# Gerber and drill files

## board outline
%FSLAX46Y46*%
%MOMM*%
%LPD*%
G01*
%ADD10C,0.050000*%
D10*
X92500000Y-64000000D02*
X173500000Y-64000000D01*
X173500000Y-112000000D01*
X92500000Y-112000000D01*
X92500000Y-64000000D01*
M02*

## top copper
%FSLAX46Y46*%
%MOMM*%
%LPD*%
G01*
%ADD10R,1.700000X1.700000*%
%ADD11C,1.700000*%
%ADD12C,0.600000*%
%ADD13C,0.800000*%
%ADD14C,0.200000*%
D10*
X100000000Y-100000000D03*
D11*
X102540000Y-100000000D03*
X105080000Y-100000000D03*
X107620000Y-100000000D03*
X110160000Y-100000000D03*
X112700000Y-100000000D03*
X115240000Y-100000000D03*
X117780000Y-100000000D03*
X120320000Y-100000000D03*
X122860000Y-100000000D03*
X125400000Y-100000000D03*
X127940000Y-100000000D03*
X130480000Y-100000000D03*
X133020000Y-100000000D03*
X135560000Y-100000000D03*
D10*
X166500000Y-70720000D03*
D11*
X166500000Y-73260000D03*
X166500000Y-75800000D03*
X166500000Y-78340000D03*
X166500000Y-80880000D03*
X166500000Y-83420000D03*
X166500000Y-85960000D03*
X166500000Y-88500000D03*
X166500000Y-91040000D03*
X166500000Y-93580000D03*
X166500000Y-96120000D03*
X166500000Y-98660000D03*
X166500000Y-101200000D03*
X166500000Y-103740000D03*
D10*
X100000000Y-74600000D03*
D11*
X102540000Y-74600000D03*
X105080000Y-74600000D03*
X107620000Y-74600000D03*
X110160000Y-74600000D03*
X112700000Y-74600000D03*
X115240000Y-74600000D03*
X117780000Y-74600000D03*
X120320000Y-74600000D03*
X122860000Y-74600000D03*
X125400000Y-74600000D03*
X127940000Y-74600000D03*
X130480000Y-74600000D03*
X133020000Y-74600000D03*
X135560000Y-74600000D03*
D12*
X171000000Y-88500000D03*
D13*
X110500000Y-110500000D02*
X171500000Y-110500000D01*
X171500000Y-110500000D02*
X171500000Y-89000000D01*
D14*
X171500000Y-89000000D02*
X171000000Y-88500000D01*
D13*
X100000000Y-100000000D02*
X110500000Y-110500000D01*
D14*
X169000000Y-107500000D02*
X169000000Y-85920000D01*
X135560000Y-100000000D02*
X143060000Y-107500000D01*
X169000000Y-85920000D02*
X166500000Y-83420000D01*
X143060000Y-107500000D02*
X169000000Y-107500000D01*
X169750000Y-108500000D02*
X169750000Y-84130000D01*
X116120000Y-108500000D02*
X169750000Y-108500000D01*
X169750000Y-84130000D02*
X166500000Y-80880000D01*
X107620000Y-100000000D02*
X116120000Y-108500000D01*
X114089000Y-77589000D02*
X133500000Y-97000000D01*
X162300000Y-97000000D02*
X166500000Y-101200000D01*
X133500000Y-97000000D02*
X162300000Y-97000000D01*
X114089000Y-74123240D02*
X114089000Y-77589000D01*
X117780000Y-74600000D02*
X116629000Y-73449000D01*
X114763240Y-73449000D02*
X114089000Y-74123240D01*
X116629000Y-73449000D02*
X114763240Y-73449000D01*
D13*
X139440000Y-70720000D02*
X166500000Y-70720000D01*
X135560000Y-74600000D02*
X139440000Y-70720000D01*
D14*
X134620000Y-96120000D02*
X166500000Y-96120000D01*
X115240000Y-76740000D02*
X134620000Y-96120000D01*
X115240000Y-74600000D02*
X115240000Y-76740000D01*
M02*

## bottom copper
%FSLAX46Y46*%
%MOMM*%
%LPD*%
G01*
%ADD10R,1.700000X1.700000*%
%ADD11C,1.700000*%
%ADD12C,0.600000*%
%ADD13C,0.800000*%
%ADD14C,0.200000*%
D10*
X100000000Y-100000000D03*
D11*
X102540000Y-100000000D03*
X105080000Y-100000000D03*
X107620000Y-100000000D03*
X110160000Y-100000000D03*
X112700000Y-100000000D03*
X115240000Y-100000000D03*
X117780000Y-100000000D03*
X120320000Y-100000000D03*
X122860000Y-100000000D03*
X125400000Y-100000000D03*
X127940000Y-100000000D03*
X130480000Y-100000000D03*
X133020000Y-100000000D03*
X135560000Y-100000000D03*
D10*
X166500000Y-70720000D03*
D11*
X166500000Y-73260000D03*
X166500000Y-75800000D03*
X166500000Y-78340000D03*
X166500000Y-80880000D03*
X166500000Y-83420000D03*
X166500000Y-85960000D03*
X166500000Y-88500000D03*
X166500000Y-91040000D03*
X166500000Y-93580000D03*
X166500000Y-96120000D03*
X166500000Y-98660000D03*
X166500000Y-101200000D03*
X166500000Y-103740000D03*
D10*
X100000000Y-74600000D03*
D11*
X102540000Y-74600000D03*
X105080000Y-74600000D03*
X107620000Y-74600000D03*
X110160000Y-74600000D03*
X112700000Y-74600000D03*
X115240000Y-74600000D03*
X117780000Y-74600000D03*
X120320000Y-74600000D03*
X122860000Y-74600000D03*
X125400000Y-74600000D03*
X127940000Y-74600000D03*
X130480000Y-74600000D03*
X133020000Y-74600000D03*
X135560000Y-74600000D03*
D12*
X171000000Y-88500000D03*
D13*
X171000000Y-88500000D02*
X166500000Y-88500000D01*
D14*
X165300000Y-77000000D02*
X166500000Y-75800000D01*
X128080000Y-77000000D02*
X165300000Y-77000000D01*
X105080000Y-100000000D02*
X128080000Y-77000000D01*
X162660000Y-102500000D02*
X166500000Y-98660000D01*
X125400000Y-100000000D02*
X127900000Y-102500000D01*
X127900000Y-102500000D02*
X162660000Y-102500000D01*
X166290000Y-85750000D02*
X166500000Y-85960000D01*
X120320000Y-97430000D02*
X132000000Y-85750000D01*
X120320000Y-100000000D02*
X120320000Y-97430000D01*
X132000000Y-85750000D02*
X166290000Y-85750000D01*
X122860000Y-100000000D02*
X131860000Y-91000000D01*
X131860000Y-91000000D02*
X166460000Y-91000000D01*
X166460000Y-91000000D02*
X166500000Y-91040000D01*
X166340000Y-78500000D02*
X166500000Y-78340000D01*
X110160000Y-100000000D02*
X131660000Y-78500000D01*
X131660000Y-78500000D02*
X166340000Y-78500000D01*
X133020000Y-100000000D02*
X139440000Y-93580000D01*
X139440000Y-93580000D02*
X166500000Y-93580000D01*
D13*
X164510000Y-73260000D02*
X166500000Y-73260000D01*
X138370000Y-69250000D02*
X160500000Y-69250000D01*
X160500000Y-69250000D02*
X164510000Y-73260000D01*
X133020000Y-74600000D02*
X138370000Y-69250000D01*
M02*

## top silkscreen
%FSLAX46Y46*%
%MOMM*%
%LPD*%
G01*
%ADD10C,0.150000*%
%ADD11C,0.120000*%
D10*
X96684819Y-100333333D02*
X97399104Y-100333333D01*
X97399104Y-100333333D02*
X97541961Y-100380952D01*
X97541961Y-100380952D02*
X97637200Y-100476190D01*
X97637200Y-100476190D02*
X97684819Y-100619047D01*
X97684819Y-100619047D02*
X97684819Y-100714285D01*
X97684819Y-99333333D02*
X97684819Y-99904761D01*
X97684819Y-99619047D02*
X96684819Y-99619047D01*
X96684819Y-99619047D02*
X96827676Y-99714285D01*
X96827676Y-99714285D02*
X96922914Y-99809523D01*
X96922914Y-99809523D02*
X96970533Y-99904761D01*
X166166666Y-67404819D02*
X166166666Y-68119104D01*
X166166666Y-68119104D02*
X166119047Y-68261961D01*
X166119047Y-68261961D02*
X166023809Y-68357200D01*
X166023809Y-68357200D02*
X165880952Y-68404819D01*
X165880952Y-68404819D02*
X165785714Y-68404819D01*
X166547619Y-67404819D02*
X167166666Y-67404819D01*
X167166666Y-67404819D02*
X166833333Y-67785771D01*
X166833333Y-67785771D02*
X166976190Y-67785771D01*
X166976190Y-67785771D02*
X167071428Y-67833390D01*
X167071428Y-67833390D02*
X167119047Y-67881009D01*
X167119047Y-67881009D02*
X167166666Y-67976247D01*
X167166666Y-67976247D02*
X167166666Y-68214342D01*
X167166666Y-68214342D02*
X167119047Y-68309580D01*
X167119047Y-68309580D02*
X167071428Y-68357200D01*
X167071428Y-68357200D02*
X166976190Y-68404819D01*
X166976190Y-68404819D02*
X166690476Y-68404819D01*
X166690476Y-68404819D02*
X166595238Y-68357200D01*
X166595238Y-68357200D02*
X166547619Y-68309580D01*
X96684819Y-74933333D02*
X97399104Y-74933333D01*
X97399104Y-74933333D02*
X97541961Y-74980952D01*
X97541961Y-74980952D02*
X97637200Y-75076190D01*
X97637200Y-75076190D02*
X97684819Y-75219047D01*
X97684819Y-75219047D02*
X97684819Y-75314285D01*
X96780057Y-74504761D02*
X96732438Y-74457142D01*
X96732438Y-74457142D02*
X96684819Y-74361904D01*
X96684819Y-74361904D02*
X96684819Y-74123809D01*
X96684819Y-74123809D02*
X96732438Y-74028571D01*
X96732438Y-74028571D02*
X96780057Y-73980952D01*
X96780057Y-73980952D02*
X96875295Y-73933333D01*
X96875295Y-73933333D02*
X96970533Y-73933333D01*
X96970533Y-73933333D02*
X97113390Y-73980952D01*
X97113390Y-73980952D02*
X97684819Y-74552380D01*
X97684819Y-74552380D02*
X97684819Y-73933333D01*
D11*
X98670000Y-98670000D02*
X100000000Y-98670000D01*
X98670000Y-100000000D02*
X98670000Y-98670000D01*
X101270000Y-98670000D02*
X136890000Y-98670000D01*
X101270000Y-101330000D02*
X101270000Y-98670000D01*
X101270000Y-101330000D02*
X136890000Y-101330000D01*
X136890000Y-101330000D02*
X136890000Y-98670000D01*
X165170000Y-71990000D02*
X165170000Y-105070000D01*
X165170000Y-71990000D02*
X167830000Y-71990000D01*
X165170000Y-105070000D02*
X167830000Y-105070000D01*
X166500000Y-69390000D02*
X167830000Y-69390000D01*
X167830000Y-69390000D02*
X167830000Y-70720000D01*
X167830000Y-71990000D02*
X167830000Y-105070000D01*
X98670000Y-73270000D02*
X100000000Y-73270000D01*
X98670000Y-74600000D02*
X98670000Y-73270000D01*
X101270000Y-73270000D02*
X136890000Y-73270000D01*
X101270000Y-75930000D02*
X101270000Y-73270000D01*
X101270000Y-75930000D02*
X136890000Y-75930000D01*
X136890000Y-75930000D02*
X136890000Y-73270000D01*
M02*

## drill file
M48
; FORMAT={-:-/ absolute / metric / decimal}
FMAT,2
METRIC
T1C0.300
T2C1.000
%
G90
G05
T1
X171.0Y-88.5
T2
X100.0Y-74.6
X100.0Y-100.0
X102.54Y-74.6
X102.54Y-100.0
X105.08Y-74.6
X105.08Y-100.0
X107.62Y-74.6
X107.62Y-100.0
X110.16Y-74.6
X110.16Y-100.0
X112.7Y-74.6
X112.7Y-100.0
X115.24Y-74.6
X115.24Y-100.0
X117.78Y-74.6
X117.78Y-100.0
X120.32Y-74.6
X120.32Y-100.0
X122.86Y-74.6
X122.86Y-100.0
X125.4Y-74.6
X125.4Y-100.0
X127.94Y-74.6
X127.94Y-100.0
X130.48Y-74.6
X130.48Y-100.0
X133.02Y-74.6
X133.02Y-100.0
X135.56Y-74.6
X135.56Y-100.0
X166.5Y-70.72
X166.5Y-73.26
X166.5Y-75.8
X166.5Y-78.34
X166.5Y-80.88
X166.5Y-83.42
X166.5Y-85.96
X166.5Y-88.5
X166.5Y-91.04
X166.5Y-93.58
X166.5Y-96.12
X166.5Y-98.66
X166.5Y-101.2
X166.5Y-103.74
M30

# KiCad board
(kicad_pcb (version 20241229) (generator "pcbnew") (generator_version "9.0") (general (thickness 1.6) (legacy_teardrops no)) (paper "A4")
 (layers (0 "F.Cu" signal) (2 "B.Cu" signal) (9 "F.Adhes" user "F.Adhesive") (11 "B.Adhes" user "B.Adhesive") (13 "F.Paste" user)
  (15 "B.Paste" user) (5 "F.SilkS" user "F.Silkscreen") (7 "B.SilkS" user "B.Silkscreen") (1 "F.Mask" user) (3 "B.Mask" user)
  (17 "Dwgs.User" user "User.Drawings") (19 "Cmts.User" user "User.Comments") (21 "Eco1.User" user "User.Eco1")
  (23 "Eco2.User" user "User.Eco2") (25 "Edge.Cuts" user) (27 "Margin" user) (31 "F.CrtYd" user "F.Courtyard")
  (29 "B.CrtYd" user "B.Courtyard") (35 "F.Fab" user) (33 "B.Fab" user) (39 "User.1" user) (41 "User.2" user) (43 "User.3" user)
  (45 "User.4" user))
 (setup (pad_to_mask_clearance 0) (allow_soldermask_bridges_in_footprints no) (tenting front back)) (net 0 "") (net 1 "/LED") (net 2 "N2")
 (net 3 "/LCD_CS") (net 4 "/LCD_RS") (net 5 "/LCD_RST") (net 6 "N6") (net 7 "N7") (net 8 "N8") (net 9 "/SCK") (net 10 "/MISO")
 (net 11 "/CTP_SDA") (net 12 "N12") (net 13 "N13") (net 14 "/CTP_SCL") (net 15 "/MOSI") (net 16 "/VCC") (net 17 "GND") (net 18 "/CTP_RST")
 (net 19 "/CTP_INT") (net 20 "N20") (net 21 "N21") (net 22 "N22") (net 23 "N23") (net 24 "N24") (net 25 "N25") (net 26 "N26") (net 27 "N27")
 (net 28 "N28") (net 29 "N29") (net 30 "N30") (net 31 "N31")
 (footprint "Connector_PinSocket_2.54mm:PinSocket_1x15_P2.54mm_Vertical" (layer "F.Cu") (at 100 100 90)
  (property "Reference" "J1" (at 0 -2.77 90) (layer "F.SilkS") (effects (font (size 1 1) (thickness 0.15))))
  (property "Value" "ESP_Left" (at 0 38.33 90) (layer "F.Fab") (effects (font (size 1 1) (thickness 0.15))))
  (fp_line (start 1.33 -1.33) (end 1.33 0) (stroke (width 0.12) (type solid)) (layer "F.SilkS"))
  (fp_line (start 0 -1.33) (end 1.33 -1.33) (stroke (width 0.12) (type solid)) (layer "F.SilkS"))
  (fp_line (start 1.33 1.27) (end 1.33 36.89) (stroke (width 0.12) (type solid)) (layer "F.SilkS"))
  (fp_line (start -1.33 1.27) (end 1.33 1.27) (stroke (width 0.12) (type solid)) (layer "F.SilkS"))
  (fp_line (start -1.33 1.27) (end -1.33 36.89) (stroke (width 0.12) (type solid)) (layer "F.SilkS"))
  (fp_line (start -1.33 36.89) (end 1.33 36.89) (stroke (width 0.12) (type solid)) (layer "F.SilkS"))
  (pad "1" thru_hole rect (at 0 0 90) (size 1.7 1.7) (drill 1) (layers "*.Cu" "*.Mask") (remove_unused_layers no) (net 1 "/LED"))
  (pad "2" thru_hole circle (at 0 2.54 90) (size 1.7 1.7) (drill 1) (layers "*.Cu" "*.Mask") (remove_unused_layers no) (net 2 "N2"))
  (pad "3" thru_hole circle (at 0 5.08 90) (size 1.7 1.7) (drill 1) (layers "*.Cu" "*.Mask") (remove_unused_layers no) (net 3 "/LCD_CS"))
  (pad "4" thru_hole circle (at 0 7.62 90) (size 1.7 1.7) (drill 1) (layers "*.Cu" "*.Mask") (remove_unused_layers no) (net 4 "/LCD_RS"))
  (pad "5" thru_hole circle (at 0 10.16 90) (size 1.7 1.7) (drill 1) (layers "*.Cu" "*.Mask") (remove_unused_layers no) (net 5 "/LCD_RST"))
  (pad "6" thru_hole circle (at 0 12.7 90) (size 1.7 1.7) (drill 1) (layers "*.Cu" "*.Mask") (remove_unused_layers no) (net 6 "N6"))
  (pad "7" thru_hole circle (at 0 15.24 90) (size 1.7 1.7) (drill 1) (layers "*.Cu" "*.Mask") (remove_unused_layers no) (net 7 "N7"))
  (pad "8" thru_hole circle (at 0 17.78 90) (size 1.7 1.7) (drill 1) (layers "*.Cu" "*.Mask") (remove_unused_layers no) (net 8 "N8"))
  (pad "9" thru_hole circle (at 0 20.32 90) (size 1.7 1.7) (drill 1) (layers "*.Cu" "*.Mask") (remove_unused_layers no) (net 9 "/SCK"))
  (pad "10" thru_hole circle (at 0 22.86 90) (size 1.7 1.7) (drill 1) (layers "*.Cu" "*.Mask") (remove_unused_layers no) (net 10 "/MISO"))
  (pad "11" thru_hole circle (at 0 25.4 90) (size 1.7 1.7) (drill 1) (layers "*.Cu" "*.Mask") (remove_unused_layers no) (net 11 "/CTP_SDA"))
  (pad "12" thru_hole circle (at 0 27.94 90) (size 1.7 1.7) (drill 1) (layers "*.Cu" "*.Mask") (remove_unused_layers no) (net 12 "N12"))
  (pad "13" thru_hole circle (at 0 30.48 90) (size 1.7 1.7) (drill 1) (layers "*.Cu" "*.Mask") (remove_unused_layers no) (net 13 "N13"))
  (pad "14" thru_hole circle (at 0 33.02 90) (size 1.7 1.7) (drill 1) (layers "*.Cu" "*.Mask") (remove_unused_layers no) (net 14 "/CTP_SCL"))
  (pad "15" thru_hole circle (at 0 35.56 90) (size 1.7 1.7) (drill 1) (layers "*.Cu" "*.Mask") (remove_unused_layers no) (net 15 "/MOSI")))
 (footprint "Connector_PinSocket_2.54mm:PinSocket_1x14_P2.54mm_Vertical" (layer "F.Cu") (at 166.5 70.72)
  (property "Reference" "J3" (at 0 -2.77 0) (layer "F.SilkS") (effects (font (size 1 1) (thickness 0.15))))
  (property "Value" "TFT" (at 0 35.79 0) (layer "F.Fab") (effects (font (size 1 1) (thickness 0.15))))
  (fp_line (start -1.33 1.27) (end -1.33 34.35) (stroke (width 0.12) (type solid)) (layer "F.SilkS"))
  (fp_line (start -1.33 1.27) (end 1.33 1.27) (stroke (width 0.12) (type solid)) (layer "F.SilkS"))
  (fp_line (start -1.33 34.35) (end 1.33 34.35) (stroke (width 0.12) (type solid)) (layer "F.SilkS"))
  (fp_line (start 0 -1.33) (end 1.33 -1.33) (stroke (width 0.12) (type solid)) (layer "F.SilkS"))
  (fp_line (start 1.33 -1.33) (end 1.33 0) (stroke (width 0.12) (type solid)) (layer "F.SilkS"))
  (fp_line (start 1.33 1.27) (end 1.33 34.35) (stroke (width 0.12) (type solid)) (layer "F.SilkS"))
  (pad "1" thru_hole rect (at 0 0) (size 1.7 1.7) (drill 1) (layers "*.Cu" "*.Mask") (remove_unused_layers no) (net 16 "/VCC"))
  (pad "2" thru_hole circle (at 0 2.54) (size 1.7 1.7) (drill 1) (layers "*.Cu" "*.Mask") (remove_unused_layers no) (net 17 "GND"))
  (pad "3" thru_hole circle (at 0 5.08) (size 1.7 1.7) (drill 1) (layers "*.Cu" "*.Mask") (remove_unused_layers no) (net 3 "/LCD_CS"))
  (pad "4" thru_hole circle (at 0 7.62) (size 1.7 1.7) (drill 1) (layers "*.Cu" "*.Mask") (remove_unused_layers no) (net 5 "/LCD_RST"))
  (pad "5" thru_hole circle (at 0 10.16) (size 1.7 1.7) (drill 1) (layers "*.Cu" "*.Mask") (remove_unused_layers no) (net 4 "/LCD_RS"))
  (pad "6" thru_hole circle (at 0 12.7) (size 1.7 1.7) (drill 1) (layers "*.Cu" "*.Mask") (remove_unused_layers no) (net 15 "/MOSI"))
  (pad "7" thru_hole circle (at 0 15.24) (size 1.7 1.7) (drill 1) (layers "*.Cu" "*.Mask") (remove_unused_layers no) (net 9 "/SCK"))
  (pad "8" thru_hole circle (at 0 17.78) (size 1.7 1.7) (drill 1) (layers "*.Cu" "*.Mask") (remove_unused_layers no) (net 1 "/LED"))
  (pad "9" thru_hole circle (at 0 20.32) (size 1.7 1.7) (drill 1) (layers "*.Cu" "*.Mask") (remove_unused_layers no) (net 10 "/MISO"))
  (pad "10" thru_hole circle (at 0 22.86) (size 1.7 1.7) (drill 1) (layers "*.Cu" "*.Mask") (remove_unused_layers no) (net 14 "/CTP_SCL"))
  (pad "11" thru_hole circle (at 0 25.4) (size 1.7 1.7) (drill 1) (layers "*.Cu" "*.Mask") (remove_unused_layers no) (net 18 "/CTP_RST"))
  (pad "12" thru_hole circle (at 0 27.94) (size 1.7 1.7) (drill 1) (layers "*.Cu" "*.Mask") (remove_unused_layers no) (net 11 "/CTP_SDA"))
  (pad "13" thru_hole circle (at 0 30.48) (size 1.7 1.7) (drill 1) (layers "*.Cu" "*.Mask") (remove_unused_layers no) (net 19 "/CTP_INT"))
  (pad "14" thru_hole circle (at 0 33.02) (size 1.7 1.7) (drill 1) (layers "*.Cu" "*.Mask") (remove_unused_layers no) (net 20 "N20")))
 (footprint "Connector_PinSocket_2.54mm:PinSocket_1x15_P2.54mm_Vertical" (layer "F.Cu") (at 100 74.6 90)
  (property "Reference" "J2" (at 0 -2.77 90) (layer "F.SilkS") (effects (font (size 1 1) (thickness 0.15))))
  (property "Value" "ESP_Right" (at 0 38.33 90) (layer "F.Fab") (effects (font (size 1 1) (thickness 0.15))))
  (fp_line (start 1.33 -1.33) (end 1.33 0) (stroke (width 0.12) (type solid)) (layer "F.SilkS"))
  (fp_line (start 0 -1.33) (end 1.33 -1.33) (stroke (width 0.12) (type solid)) (layer "F.SilkS"))
  (fp_line (start 1.33 1.27) (end 1.33 36.89) (stroke (width 0.12) (type solid)) (layer "F.SilkS"))
  (fp_line (start -1.33 1.27) (end 1.33 1.27) (stroke (width 0.12) (type solid)) (layer "F.SilkS"))
  (fp_line (start -1.33 1.27) (end -1.33 36.89) (stroke (width 0.12) (type solid)) (layer "F.SilkS"))
  (fp_line (start -1.33 36.89) (end 1.33 36.89) (stroke (width 0.12) (type solid)) (layer "F.SilkS"))
  (pad "1" thru_hole rect (at 0 0 90) (size 1.7 1.7) (drill 1) (layers "*.Cu" "*.Mask") (remove_unused_layers no) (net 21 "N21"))
  (pad "2" thru_hole circle (at 0 2.54 90) (size 1.7 1.7) (drill 1) (layers "*.Cu" "*.Mask") (remove_unused_layers no) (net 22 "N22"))
  (pad "3" thru_hole circle (at 0 5.08 90) (size 1.7 1.7) (drill 1) (layers "*.Cu" "*.Mask") (remove_unused_layers no) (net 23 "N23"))
  (pad "4" thru_hole circle (at 0 7.62 90) (size 1.7 1.7) (drill 1) (layers "*.Cu" "*.Mask") (remove_unused_layers no) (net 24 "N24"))
  (pad "5" thru_hole circle (at 0 10.16 90) (size 1.7 1.7) (drill 1) (layers "*.Cu" "*.Mask") (remove_unused_layers no) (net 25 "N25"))
  (pad "6" thru_hole circle (at 0 12.7 90) (size 1.7 1.7) (drill 1) (layers "*.Cu" "*.Mask") (remove_unused_layers no) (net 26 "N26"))
  (pad "7" thru_hole circle (at 0 15.24 90) (size 1.7 1.7) (drill 1) (layers "*.Cu" "*.Mask") (remove_unused_layers no) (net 18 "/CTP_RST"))
  (pad "8" thru_hole circle (at 0 17.78 90) (size 1.7 1.7) (drill 1) (layers "*.Cu" "*.Mask") (remove_unused_layers no) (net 19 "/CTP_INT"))
  (pad "9" thru_hole circle (at 0 20.32 90) (size 1.7 1.7) (drill 1) (layers "*.Cu" "*.Mask") (remove_unused_layers no) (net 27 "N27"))
  (pad "10" thru_hole circle (at 0 22.86 90) (size 1.7 1.7) (drill 1) (layers "*.Cu" "*.Mask") (remove_unused_layers no) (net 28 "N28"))
  (pad "11" thru_hole circle (at 0 25.4 90) (size 1.7 1.7) (drill 1) (layers "*.Cu" "*.Mask") (remove_unused_layers no) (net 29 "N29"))
  (pad "12" thru_hole circle (at 0 27.94 90) (size 1.7 1.7) (drill 1) (layers "*.Cu" "*.Mask") (remove_unused_layers no) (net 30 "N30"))
  (pad "13" thru_hole circle (at 0 30.48 90) (size 1.7 1.7) (drill 1) (layers "*.Cu" "*.Mask") (remove_unused_layers no) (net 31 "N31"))
  (pad "14" thru_hole circle (at 0 33.02 90) (size 1.7 1.7) (drill 1) (layers "*.Cu" "*.Mask") (remove_unused_layers no) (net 17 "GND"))
  (pad "15" thru_hole circle (at 0 35.56 90) (size 1.7 1.7) (drill 1) (layers "*.Cu" "*.Mask") (remove_unused_layers no) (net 16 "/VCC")))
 (gr_rect (start 92.5 64) (end 173.5 112) (stroke (width 0.05) (type default)) (fill no) (layer "Edge.Cuts"))
 (segment (start 110.5 110.5) (end 171.5 110.5) (width 0.8) (layer "F.Cu") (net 1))
 (segment (start 171.5 110.5) (end 171.5 89) (width 0.8) (layer "F.Cu") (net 1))
 (segment (start 171.5 89) (end 171 88.5) (width 0.2) (layer "F.Cu") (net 1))
 (segment (start 100 100) (end 110.5 110.5) (width 0.8) (layer "F.Cu") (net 1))
 (via (at 171 88.5) (size 0.6) (drill 0.3) (layers "F.Cu" "B.Cu") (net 1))
 (segment (start 171 88.5) (end 166.5 88.5) (width 0.8) (layer "B.Cu") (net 1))
 (segment (start 165.3 77) (end 166.5 75.8) (width 0.2) (layer "B.Cu") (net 3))
 (segment (start 128.08 77) (end 165.3 77) (width 0.2) (layer "B.Cu") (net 3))
 (segment (start 105.08 100) (end 128.08 77) (width 0.2) (layer "B.Cu") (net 3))
 (segment (start 169 107.5) (end 169 85.92) (width 0.2) (layer "F.Cu") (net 15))
 (segment (start 135.56 100) (end 143.06 107.5) (width 0.2) (layer "F.Cu") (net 15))
 (segment (start 169 85.92) (end 166.5 83.42) (width 0.2) (layer "F.Cu") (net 15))
 (segment (start 143.06 107.5) (end 169 107.5) (width 0.2) (layer "F.Cu") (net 15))
 (segment (start 162.66 102.5) (end 166.5 98.66) (width 0.2) (layer "B.Cu") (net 11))
 (segment (start 125.4 100) (end 127.9 102.5) (width 0.2) (layer "B.Cu") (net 11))
 (segment (start 127.9 102.5) (end 162.66 102.5) (width 0.2) (layer "B.Cu") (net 11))
 (segment (start 166.29 85.75) (end 166.5 85.96) (width 0.2) (layer "B.Cu") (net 9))
 (segment (start 120.32 97.43) (end 132 85.75) (width 0.2) (layer "B.Cu") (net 9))
 (segment (start 120.32 100) (end 120.32 97.43) (width 0.2) (layer "B.Cu") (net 9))
 (segment (start 132 85.75) (end 166.29 85.75) (width 0.2) (layer "B.Cu") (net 9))
 (segment (start 122.86 100) (end 131.86 91) (width 0.2) (layer "B.Cu") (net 10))
 (segment (start 131.86 91) (end 166.46 91) (width 0.2) (layer "B.Cu") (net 10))
 (segment (start 166.46 91) (end 166.5 91.04) (width 0.2) (layer "B.Cu") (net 10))
 (segment (start 169.75 108.5) (end 169.75 84.13) (width 0.2) (layer "F.Cu") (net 4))
 (segment (start 116.12 108.5) (end 169.75 108.5) (width 0.2) (layer "F.Cu") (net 4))
 (segment (start 169.75 84.13) (end 166.5 80.88) (width 0.2) (layer "F.Cu") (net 4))
 (segment (start 107.62 100) (end 116.12 108.5) (width 0.2) (layer "F.Cu") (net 4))
 (segment (start 166.34 78.5) (end 166.5 78.34) (width 0.2) (layer "B.Cu") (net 5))
 (segment (start 110.16 100) (end 131.66 78.5) (width 0.2) (layer "B.Cu") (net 5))
 (segment (start 131.66 78.5) (end 166.34 78.5) (width 0.2) (layer "B.Cu") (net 5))
 (segment (start 133.02 100) (end 139.44 93.58) (width 0.2) (layer "B.Cu") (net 14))
 (segment (start 139.44 93.58) (end 166.5 93.58) (width 0.2) (layer "B.Cu") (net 14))
 (segment (start 164.51 73.26) (end 166.5 73.26) (width 0.8) (layer "B.Cu") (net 17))
 (segment (start 138.37 69.25) (end 160.5 69.25) (width 0.8) (layer "B.Cu") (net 17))
 (segment (start 160.5 69.25) (end 164.51 73.26) (width 0.8) (layer "B.Cu") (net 17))
 (segment (start 133.02 74.6) (end 138.37 69.25) (width 0.8) (layer "B.Cu") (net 17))
 (segment (start 114.089 77.589) (end 133.5 97) (width 0.2) (layer "F.Cu") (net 19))
 (segment (start 162.3 97) (end 166.5 101.2) (width 0.2) (layer "F.Cu") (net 19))
 (segment (start 133.5 97) (end 162.3 97) (width 0.2) (layer "F.Cu") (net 19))
 (segment (start 114.089 74.12324) (end 114.089 77.589) (width 0.2) (layer "F.Cu") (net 19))
 (segment (start 117.78 74.6) (end 116.629 73.449) (width 0.2) (layer "F.Cu") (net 19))
 (segment (start 114.76324 73.449) (end 114.089 74.12324) (width 0.2) (layer "F.Cu") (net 19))
 (segment (start 116.629 73.449) (end 114.76324 73.449) (width 0.2) (layer "F.Cu") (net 19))
 (segment (start 139.44 70.72) (end 166.5 70.72) (width 0.8) (layer "F.Cu") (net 16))
 (segment (start 135.56 74.6) (end 139.44 70.72) (width 0.8) (layer "F.Cu") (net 16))
 (segment (start 134.62 96.12) (end 166.5 96.12) (width 0.2) (layer "F.Cu") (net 18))
 (segment (start 115.24 76.74) (end 134.62 96.12) (width 0.2) (layer "F.Cu") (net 18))
 (segment (start 115.24 74.6) (end 115.24 76.74) (width 0.2) (layer "F.Cu") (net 18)))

